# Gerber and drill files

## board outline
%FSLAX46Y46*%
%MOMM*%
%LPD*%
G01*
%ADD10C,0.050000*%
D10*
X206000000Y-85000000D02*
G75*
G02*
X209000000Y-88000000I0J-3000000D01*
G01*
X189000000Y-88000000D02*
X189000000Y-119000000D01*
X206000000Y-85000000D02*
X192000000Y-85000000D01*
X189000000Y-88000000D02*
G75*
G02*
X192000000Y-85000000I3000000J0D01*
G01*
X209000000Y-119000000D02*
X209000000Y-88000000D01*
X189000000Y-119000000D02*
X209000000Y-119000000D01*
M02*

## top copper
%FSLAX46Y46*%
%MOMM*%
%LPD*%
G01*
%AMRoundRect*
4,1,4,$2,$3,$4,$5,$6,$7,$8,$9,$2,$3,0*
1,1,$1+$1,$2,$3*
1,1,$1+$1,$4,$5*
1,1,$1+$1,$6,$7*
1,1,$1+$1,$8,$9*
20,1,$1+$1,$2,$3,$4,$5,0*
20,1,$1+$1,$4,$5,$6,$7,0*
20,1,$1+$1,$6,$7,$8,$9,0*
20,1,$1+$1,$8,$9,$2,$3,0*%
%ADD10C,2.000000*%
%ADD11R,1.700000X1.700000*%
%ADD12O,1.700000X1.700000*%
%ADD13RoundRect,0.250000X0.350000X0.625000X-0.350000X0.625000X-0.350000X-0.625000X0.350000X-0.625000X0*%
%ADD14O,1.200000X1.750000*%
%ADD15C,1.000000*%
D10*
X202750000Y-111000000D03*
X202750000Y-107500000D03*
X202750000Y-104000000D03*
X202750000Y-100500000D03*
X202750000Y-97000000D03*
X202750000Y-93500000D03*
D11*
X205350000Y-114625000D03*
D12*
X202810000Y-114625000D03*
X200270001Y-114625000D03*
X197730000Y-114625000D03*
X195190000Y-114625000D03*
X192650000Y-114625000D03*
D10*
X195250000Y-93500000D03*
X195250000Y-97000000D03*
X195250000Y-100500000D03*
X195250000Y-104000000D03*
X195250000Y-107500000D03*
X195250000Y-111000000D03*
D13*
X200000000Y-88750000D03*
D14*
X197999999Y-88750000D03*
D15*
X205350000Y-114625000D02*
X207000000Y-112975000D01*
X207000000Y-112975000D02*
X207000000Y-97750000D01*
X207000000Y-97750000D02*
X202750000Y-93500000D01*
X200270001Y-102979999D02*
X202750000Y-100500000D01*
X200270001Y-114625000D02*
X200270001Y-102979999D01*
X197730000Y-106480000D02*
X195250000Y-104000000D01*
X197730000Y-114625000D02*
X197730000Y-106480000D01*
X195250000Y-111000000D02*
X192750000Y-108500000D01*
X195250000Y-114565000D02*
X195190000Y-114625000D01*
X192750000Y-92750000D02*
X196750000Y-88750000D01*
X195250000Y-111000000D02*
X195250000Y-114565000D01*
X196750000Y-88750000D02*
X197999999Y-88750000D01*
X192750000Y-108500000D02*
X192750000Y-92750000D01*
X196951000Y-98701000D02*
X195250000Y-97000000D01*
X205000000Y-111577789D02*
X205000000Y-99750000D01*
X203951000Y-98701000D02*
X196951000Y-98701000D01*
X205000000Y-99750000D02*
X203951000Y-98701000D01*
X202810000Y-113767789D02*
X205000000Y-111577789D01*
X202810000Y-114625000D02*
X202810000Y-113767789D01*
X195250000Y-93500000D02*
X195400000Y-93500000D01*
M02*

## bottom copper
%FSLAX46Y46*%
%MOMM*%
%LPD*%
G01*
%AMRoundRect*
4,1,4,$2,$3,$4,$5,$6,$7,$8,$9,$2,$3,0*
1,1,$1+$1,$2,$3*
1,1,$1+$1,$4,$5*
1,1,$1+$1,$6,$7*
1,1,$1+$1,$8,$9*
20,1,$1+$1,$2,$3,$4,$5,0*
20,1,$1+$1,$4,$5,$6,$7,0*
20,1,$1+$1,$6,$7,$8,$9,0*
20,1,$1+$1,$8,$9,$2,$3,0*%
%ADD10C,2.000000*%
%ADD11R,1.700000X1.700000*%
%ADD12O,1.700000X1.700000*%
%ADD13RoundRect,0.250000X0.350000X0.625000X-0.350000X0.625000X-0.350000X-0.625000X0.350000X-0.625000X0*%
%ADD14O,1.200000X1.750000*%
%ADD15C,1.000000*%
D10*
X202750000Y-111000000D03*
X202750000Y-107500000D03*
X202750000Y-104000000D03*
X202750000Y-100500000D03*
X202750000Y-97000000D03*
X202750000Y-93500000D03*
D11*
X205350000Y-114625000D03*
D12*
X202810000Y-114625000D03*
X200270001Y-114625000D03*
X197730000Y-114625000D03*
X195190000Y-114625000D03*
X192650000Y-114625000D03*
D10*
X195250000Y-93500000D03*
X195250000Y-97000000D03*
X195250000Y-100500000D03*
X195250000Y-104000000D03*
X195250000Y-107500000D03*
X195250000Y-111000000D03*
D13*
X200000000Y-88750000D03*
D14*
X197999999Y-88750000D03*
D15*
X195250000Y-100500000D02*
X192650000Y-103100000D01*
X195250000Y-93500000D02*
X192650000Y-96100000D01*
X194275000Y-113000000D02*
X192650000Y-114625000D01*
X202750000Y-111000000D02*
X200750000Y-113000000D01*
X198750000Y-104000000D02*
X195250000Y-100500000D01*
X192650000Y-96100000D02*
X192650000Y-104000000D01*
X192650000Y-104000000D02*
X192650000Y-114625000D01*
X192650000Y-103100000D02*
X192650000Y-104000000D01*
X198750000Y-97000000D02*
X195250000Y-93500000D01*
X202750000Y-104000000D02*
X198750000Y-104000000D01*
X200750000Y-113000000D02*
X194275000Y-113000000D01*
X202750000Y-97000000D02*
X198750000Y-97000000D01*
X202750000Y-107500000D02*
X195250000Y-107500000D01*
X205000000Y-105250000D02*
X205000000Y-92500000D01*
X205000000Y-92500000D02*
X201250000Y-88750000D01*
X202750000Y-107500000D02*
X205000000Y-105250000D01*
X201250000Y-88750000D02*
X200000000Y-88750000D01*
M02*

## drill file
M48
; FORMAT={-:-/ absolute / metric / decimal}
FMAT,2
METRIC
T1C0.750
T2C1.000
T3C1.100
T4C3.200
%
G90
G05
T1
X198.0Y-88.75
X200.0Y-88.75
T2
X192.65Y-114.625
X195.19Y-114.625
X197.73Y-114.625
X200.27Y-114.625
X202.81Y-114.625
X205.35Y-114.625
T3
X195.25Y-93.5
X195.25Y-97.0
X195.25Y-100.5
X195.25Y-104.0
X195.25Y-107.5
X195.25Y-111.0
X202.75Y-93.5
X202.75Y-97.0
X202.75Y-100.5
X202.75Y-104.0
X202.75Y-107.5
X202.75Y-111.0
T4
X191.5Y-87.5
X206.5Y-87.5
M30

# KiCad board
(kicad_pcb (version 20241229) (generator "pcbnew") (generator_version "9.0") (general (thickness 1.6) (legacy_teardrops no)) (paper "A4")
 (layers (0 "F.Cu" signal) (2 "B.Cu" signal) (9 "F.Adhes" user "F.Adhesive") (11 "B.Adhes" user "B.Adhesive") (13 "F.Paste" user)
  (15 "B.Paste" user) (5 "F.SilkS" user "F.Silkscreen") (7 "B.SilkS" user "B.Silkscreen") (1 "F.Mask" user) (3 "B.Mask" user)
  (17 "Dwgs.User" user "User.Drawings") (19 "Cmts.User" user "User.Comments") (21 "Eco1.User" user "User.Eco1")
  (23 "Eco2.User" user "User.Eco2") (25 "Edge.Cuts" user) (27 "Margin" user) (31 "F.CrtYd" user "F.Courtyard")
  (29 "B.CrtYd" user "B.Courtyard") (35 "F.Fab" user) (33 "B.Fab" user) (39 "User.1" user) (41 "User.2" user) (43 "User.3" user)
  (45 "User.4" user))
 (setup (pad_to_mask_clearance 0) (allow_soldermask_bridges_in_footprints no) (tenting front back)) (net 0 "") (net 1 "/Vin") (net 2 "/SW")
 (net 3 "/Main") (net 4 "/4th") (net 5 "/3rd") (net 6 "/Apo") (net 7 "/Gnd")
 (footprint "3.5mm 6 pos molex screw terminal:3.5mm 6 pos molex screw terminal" (layer "F.Cu") (at 202.75 111 90)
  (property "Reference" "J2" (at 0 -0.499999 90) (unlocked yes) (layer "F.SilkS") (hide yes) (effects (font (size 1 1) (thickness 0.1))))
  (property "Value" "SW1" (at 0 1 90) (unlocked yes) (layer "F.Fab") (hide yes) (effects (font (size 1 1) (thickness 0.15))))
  (pad "1" thru_hole circle (at 0 0 90) (size 2 2) (drill 1.1) (layers "*.Cu" "*.Mask") (remove_unused_layers no) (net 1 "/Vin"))
  (pad "2" thru_hole circle (at 3.5 0 90) (size 2 2) (drill 1.1) (layers "*.Cu" "*.Mask") (remove_unused_layers no) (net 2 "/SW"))
  (pad "3" thru_hole circle (at 7 0 90) (size 2 2) (drill 1.1) (layers "*.Cu" "*.Mask") (remove_unused_layers no) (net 1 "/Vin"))
  (pad "4" thru_hole circle (at 10.5 0 90) (size 2 2) (drill 1.1) (layers "*.Cu" "*.Mask") (remove_unused_layers no) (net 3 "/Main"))
  (pad "5" thru_hole circle (at 14 0 90) (size 2 2) (drill 1.1) (layers "*.Cu" "*.Mask") (remove_unused_layers no) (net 1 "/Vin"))
  (pad "6" thru_hole circle (at 17.5 0 90) (size 2 2) (drill 1.1) (layers "*.Cu" "*.Mask") (remove_unused_layers no) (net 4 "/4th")))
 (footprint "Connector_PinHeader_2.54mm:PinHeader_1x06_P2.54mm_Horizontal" (layer "F.Cu") (at 205.35 114.625 -90)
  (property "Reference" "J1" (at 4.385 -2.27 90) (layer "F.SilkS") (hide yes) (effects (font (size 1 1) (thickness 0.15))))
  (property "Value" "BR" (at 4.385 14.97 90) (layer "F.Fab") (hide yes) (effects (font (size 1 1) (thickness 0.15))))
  (pad "1" thru_hole rect (at 0 0 270) (size 1.7 1.7) (drill 1) (layers "*.Cu" "*.Mask") (remove_unused_layers no) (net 4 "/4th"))
  (pad "2" thru_hole oval (at 0 2.54 270) (size 1.7 1.7) (drill 1) (layers "*.Cu" "*.Mask") (remove_unused_layers no) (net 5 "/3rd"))
  (pad "3" thru_hole oval (at 0 5.079999 270) (size 1.7 1.7) (drill 1) (layers "*.Cu" "*.Mask") (remove_unused_layers no) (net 3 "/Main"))
  (pad "4" thru_hole oval (at 0 7.62 270) (size 1.7 1.7) (drill 1) (layers "*.Cu" "*.Mask") (remove_unused_layers no) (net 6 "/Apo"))
  (pad "5" thru_hole oval (at 0 10.16 270) (size 1.7 1.7) (drill 1) (layers "*.Cu" "*.Mask") (remove_unused_layers no) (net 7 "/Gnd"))
  (pad "6" thru_hole oval (at 0 12.7 270) (size 1.7 1.7) (drill 1) (layers "*.Cu" "*.Mask") (remove_unused_layers no) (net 1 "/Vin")))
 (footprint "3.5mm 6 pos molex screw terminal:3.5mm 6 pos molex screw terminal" (layer "F.Cu") (at 195.25 93.5 -90)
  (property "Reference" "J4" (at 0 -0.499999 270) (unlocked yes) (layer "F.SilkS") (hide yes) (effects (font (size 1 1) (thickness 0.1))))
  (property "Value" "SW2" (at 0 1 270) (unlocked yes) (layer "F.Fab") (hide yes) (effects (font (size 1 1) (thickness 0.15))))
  (pad "1" thru_hole circle (at 0 0 270) (size 2 2) (drill 1.1) (layers "*.Cu" "*.Mask") (remove_unused_layers no) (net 1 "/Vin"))
  (pad "2" thru_hole circle (at 3.5 0 270) (size 2 2) (drill 1.1) (layers "*.Cu" "*.Mask") (remove_unused_layers no) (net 5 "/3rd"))
  (pad "3" thru_hole circle (at 7 0 270) (size 2 2) (drill 1.1) (layers "*.Cu" "*.Mask") (remove_unused_layers no) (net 1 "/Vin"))
  (pad "4" thru_hole circle (at 10.5 0 270) (size 2 2) (drill 1.1) (layers "*.Cu" "*.Mask") (remove_unused_layers no) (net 6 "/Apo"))
  (pad "5" thru_hole circle (at 14 0 270) (size 2 2) (drill 1.1) (layers "*.Cu" "*.Mask") (remove_unused_layers no) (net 2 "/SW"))
  (pad "6" thru_hole circle (at 17.5 0 270) (size 2 2) (drill 1.1) (layers "*.Cu" "*.Mask") (remove_unused_layers no) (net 7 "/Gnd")))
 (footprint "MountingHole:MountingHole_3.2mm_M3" (layer "F.Cu") (at 206.5 87.5)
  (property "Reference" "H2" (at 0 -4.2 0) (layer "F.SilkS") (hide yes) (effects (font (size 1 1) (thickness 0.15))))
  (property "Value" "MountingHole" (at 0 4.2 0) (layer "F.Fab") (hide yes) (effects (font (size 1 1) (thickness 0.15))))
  (pad "" np_thru_hole circle (at 0 0) (size 3.2 3.2) (drill 3.2) (layers "*.Cu" "*.Mask")))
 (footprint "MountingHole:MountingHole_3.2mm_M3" (layer "F.Cu") (at 191.5 87.5)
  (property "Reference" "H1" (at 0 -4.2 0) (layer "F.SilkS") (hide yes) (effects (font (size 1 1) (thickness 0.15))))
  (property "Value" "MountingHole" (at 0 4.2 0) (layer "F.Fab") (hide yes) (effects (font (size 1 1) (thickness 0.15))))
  (pad "" np_thru_hole circle (at 0 0) (size 3.2 3.2) (drill 3.2) (layers "*.Cu" "*.Mask")))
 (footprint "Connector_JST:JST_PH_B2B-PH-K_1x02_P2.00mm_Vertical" (layer "F.Cu") (at 200 88.75 180)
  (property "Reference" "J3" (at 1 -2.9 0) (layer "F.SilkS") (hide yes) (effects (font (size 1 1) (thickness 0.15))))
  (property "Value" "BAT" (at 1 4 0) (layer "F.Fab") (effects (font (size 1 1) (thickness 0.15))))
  (pad "1" thru_hole roundrect (at 0 0 180) (size 1.2 1.75) (drill 0.75) (layers "*.Cu" "*.Mask") (remove_unused_layers no)
   (roundrect_rratio 0.208333) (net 2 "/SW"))
  (pad "2" thru_hole oval (at 2.000001 0 180) (size 1.2 1.75) (drill 0.75) (layers "*.Cu" "*.Mask") (remove_unused_layers no) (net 7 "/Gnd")))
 (gr_arc (start 206 85) (mid 208.12132 85.87868) (end 209 88) (stroke (width 0.05) (type default)) (layer "Edge.Cuts"))
 (gr_line (start 189 88) (end 189 119) (stroke (width 0.05) (type default)) (layer "Edge.Cuts"))
 (gr_line (start 206 85) (end 192 85) (stroke (width 0.05) (type default)) (layer "Edge.Cuts"))
 (gr_arc (start 189 88) (mid 189.87868 85.87868) (end 192 85) (stroke (width 0.05) (type default)) (layer "Edge.Cuts"))
 (gr_line (start 209 119) (end 209 88) (stroke (width 0.05) (type default)) (layer "Edge.Cuts"))
 (gr_line (start 189 119) (end 209 119) (stroke (width 0.05) (type default)) (layer "Edge.Cuts"))
 (segment (start 205.35 114.625) (end 207 112.975) (width 1) (layer "F.Cu") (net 4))
 (segment (start 207 112.975) (end 207 97.75) (width 1) (layer "F.Cu") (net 4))
 (segment (start 207 97.75) (end 202.75 93.5) (width 1) (layer "F.Cu") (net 4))
 (segment (start 200.270001 102.979999) (end 202.75 100.5) (width 1) (layer "F.Cu") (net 3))
 (segment (start 200.270001 114.625) (end 200.270001 102.979999) (width 1) (layer "F.Cu") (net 3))
 (segment (start 197.73 106.48) (end 195.25 104) (width 1) (layer "F.Cu") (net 6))
 (segment (start 197.73 114.625) (end 197.73 106.48) (width 1) (layer "F.Cu") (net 6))
 (segment (start 195.25 111) (end 192.75 108.5) (width 1) (layer "F.Cu") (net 7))
 (segment (start 195.25 114.565) (end 195.19 114.625) (width 1) (layer "F.Cu") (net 7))
 (segment (start 192.75 92.75) (end 196.75 88.75) (width 1) (layer "F.Cu") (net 7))
 (segment (start 195.25 111) (end 195.25 114.565) (width 1) (layer "F.Cu") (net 7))
 (segment (start 196.75 88.75) (end 197.999999 88.75) (width 1) (layer "F.Cu") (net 7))
 (segment (start 192.75 108.5) (end 192.75 92.75) (width 1) (layer "F.Cu") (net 7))
 (segment (start 196.951 98.701) (end 195.25 97) (width 1) (layer "F.Cu") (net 5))
 (segment (start 205 111.577789) (end 205 99.75) (width 1) (layer "F.Cu") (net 5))
 (segment (start 203.951 98.701) (end 196.951 98.701) (width 1) (layer "F.Cu") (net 5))
 (segment (start 205 99.75) (end 203.951 98.701) (width 1) (layer "F.Cu") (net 5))
 (segment (start 202.81 113.767789) (end 205 111.577789) (width 1) (layer "F.Cu") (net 5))
 (segment (start 202.81 114.625) (end 202.81 113.767789) (width 1) (layer "F.Cu") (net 5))
 (segment (start 195.25 93.5) (end 195.4 93.5) (width 1) (layer "F.Cu") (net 1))
 (segment (start 195.25 100.5) (end 192.65 103.1) (width 1) (layer "B.Cu") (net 1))
 (segment (start 195.25 93.5) (end 192.65 96.1) (width 1) (layer "B.Cu") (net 1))
 (segment (start 194.275 113) (end 192.65 114.625) (width 1) (layer "B.Cu") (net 1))
 (segment (start 202.75 111) (end 200.75 113) (width 1) (layer "B.Cu") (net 1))
 (segment (start 198.75 104) (end 195.25 100.5) (width 1) (layer "B.Cu") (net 1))
 (segment (start 192.65 96.1) (end 192.65 104) (width 1) (layer "B.Cu") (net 1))
 (segment (start 192.65 104) (end 192.65 114.625) (width 1) (layer "B.Cu") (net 1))
 (segment (start 192.65 103.1) (end 192.65 104) (width 1) (layer "B.Cu") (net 1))
 (segment (start 198.75 97) (end 195.25 93.5) (width 1) (layer "B.Cu") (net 1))
 (segment (start 202.75 104) (end 198.75 104) (width 1) (layer "B.Cu") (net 1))
 (segment (start 200.75 113) (end 194.275 113) (width 1) (layer "B.Cu") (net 1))
 (segment (start 202.75 97) (end 198.75 97) (width 1) (layer "B.Cu") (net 1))
 (segment (start 202.75 107.5) (end 195.25 107.5) (width 1) (layer "B.Cu") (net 2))
 (segment (start 205 105.25) (end 205 92.5) (width 1) (layer "B.Cu") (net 2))
 (segment (start 205 92.5) (end 201.25 88.75) (width 1) (layer "B.Cu") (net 2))
 (segment (start 202.75 107.5) (end 205 105.25) (width 1) (layer "B.Cu") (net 2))
 (segment (start 201.25 88.75) (end 200 88.75) (width 1) (layer "B.Cu") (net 2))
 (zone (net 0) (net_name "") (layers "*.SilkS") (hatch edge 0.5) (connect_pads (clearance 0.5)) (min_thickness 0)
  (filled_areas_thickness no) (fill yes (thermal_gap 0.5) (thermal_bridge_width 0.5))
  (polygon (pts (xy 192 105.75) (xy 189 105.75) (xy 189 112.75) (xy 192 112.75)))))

